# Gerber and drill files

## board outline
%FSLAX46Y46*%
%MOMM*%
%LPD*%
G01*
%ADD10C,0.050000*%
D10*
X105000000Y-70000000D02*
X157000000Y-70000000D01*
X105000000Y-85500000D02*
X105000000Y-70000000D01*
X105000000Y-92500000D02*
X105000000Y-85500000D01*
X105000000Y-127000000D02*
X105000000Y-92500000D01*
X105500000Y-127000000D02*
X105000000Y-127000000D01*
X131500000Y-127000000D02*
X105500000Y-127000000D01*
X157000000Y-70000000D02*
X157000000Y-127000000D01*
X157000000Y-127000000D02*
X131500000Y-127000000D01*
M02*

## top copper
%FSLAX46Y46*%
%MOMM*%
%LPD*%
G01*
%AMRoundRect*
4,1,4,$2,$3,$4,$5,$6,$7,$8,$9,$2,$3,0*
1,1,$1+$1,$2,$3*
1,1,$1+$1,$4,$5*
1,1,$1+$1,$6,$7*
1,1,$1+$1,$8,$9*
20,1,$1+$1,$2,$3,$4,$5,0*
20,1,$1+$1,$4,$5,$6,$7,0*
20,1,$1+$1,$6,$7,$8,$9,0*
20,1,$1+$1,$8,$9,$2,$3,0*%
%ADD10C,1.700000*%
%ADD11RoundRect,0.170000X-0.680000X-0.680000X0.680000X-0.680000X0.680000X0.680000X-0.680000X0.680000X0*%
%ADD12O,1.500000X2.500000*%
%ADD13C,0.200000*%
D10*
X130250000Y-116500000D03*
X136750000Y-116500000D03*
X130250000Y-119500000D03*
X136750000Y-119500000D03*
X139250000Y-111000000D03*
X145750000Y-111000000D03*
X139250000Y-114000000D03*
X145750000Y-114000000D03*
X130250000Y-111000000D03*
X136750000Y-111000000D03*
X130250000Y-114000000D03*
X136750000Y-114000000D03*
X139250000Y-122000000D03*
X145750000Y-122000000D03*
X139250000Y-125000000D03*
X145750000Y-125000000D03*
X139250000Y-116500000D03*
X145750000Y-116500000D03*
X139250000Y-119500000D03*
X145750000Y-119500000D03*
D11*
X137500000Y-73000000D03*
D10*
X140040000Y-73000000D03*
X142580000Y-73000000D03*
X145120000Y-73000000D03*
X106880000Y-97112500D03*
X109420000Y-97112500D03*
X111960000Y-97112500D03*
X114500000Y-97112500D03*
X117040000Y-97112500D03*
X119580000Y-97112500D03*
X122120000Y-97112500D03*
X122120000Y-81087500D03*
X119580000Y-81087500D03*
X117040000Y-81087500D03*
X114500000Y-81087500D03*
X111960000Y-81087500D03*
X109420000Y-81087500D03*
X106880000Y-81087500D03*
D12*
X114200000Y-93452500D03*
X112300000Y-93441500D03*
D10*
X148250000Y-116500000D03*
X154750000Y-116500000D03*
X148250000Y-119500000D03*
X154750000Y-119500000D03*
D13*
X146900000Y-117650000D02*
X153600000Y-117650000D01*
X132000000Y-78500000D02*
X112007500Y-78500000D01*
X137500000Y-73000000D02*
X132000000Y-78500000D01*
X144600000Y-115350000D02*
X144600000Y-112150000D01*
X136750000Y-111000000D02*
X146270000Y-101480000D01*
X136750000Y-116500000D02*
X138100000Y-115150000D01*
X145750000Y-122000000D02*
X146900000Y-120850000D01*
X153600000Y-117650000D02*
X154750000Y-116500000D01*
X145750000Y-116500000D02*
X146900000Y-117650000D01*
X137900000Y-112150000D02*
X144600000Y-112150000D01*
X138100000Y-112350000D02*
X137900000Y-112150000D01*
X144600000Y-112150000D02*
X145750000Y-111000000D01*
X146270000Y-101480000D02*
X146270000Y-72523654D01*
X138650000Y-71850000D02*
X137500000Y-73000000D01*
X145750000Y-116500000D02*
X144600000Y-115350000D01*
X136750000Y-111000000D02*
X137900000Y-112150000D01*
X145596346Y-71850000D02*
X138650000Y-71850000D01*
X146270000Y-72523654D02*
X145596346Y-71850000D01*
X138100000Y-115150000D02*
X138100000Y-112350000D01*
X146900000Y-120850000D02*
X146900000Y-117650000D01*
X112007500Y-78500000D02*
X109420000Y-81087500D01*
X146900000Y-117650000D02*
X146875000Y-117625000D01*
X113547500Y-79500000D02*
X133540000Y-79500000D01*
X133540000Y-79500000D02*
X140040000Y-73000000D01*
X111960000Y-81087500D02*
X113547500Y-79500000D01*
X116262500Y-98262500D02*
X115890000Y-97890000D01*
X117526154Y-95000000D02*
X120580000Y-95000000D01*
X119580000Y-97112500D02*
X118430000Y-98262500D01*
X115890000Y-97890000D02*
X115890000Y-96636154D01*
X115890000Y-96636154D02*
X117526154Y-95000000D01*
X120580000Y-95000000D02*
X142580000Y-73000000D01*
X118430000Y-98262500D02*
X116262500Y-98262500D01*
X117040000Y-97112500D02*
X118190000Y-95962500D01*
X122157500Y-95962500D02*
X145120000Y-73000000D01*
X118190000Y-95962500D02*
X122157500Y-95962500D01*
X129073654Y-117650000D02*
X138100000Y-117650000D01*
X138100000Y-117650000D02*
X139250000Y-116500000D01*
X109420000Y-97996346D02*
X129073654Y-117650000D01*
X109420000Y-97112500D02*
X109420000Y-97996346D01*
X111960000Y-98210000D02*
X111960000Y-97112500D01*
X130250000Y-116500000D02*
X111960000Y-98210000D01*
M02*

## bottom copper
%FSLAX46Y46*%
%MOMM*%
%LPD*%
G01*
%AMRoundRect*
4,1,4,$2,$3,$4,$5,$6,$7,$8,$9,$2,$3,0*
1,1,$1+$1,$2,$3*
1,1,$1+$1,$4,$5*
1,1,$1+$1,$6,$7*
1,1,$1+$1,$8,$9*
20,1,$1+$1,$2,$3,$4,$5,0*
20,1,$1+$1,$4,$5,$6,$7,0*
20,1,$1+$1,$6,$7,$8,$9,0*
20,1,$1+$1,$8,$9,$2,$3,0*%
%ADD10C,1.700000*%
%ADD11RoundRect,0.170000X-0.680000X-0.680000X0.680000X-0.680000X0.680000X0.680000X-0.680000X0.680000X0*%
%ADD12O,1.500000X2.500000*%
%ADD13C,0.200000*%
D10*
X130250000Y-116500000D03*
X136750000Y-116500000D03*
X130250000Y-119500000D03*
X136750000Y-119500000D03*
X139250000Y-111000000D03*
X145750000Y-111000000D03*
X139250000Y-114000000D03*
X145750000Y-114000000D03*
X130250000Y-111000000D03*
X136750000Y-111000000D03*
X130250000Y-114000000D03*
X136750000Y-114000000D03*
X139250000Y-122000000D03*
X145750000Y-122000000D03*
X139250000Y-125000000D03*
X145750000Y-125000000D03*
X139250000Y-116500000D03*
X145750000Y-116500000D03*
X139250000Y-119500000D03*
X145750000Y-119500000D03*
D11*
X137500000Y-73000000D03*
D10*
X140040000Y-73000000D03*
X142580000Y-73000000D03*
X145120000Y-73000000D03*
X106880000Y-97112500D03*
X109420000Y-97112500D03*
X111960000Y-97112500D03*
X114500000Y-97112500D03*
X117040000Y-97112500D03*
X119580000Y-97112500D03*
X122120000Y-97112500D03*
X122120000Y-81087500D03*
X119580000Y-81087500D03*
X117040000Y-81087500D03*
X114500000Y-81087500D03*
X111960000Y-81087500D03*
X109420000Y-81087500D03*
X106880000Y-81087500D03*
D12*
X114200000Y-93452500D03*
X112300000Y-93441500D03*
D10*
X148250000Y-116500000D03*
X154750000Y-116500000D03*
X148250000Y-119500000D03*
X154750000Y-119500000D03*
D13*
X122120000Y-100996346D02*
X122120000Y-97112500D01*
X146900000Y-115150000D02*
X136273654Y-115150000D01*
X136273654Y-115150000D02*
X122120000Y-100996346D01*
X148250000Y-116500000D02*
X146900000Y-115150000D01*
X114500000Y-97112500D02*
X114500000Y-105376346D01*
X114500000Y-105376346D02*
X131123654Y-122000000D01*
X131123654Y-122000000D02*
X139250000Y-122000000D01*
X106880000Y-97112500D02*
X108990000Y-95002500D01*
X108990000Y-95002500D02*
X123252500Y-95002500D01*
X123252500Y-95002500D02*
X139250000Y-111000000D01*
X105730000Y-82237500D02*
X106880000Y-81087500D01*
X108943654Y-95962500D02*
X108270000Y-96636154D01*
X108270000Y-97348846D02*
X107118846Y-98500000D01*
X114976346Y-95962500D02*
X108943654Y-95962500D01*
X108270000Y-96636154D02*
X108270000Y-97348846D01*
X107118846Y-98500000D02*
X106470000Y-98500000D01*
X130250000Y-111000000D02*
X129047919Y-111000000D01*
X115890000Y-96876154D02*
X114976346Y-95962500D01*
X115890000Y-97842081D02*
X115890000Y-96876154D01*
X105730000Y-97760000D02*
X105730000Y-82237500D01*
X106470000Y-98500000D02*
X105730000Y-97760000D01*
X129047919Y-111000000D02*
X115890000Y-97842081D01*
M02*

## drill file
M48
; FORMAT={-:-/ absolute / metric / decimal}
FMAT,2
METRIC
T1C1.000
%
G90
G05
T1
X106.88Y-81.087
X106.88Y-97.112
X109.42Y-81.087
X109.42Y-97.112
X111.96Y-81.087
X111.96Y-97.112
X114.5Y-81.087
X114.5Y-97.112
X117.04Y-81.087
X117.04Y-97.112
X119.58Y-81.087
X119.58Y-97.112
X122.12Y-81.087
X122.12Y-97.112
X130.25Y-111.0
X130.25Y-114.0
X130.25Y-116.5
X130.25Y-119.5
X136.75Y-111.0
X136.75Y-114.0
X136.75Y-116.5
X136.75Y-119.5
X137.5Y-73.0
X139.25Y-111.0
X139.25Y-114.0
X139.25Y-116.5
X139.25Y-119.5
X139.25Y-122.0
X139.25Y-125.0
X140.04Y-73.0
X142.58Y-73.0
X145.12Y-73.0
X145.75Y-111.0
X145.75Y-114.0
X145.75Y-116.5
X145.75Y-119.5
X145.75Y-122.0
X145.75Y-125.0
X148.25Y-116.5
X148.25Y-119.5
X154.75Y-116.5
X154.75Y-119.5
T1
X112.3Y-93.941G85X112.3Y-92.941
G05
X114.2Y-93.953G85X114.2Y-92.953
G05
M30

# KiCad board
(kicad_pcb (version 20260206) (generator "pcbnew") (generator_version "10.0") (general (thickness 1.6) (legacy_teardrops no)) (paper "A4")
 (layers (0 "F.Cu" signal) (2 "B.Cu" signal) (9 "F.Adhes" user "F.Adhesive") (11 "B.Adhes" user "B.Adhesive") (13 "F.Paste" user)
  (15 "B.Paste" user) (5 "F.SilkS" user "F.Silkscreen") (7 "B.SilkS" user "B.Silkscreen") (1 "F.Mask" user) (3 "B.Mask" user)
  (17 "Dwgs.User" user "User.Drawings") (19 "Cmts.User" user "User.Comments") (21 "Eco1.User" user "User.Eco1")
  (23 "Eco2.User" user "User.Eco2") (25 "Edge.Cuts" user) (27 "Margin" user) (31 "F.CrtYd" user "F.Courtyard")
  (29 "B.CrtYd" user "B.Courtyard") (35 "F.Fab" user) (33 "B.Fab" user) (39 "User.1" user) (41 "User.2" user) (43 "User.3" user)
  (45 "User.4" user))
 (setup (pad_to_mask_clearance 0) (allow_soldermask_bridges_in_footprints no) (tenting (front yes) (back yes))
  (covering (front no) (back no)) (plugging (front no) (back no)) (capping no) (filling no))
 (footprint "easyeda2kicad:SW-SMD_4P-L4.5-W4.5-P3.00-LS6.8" (layer "F.Cu") (at 133.5 118)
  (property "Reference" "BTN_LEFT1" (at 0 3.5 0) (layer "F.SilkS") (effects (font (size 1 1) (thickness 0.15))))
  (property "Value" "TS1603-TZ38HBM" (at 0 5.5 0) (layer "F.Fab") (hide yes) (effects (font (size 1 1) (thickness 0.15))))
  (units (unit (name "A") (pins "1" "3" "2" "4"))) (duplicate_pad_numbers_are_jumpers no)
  (pad "1" thru_hole circle (at -3.25 -1.5) (size 1.7 1.7) (drill 1) (layers "*.Cu" "*.Mask") (remove_unused_layers no)
   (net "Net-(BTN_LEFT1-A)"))
  (pad "2" thru_hole circle (at 3.25 -1.5) (size 1.7 1.7) (drill 1) (layers "*.Cu" "*.Mask") (remove_unused_layers no) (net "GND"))
  (pad "3" thru_hole circle (at -3.25 1.5) (size 1.7 1.7) (drill 1) (layers "*.Cu" "*.Mask") (remove_unused_layers no)
   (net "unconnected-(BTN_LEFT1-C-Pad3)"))
  (pad "4" thru_hole circle (at 3.25 1.5) (size 1.7 1.7) (drill 1) (layers "*.Cu" "*.Mask") (remove_unused_layers no)
   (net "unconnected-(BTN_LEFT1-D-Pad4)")))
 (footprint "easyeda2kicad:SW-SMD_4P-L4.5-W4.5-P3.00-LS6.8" (layer "F.Cu") (at 142.5 112.5)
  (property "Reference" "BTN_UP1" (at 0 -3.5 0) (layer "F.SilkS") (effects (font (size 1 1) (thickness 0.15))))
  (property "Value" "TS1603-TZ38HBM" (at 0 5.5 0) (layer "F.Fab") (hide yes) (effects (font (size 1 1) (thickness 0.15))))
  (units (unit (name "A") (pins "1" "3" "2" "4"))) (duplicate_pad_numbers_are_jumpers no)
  (pad "1" thru_hole circle (at -3.25 -1.5) (size 1.7 1.7) (drill 1) (layers "*.Cu" "*.Mask") (remove_unused_layers no)
   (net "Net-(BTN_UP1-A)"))
  (pad "2" thru_hole circle (at 3.25 -1.5) (size 1.7 1.7) (drill 1) (layers "*.Cu" "*.Mask") (remove_unused_layers no) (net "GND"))
  (pad "3" thru_hole circle (at -3.25 1.5) (size 1.7 1.7) (drill 1) (layers "*.Cu" "*.Mask") (remove_unused_layers no)
   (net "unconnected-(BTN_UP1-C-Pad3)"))
  (pad "4" thru_hole circle (at 3.25 1.5) (size 1.7 1.7) (drill 1) (layers "*.Cu" "*.Mask") (remove_unused_layers no)
   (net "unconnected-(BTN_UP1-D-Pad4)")))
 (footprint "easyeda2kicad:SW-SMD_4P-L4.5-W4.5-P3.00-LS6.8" (layer "F.Cu") (at 133.5 112.5)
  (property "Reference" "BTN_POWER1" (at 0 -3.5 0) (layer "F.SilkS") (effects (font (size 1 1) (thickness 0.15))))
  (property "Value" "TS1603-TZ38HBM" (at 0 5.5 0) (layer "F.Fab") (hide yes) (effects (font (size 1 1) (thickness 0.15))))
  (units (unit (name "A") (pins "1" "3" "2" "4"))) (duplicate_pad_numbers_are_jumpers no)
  (pad "1" thru_hole circle (at -3.25 -1.5) (size 1.7 1.7) (drill 1) (layers "*.Cu" "*.Mask") (remove_unused_layers no)
   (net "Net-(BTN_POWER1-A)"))
  (pad "2" thru_hole circle (at 3.25 -1.5) (size 1.7 1.7) (drill 1) (layers "*.Cu" "*.Mask") (remove_unused_layers no) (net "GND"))
  (pad "3" thru_hole circle (at -3.25 1.5) (size 1.7 1.7) (drill 1) (layers "*.Cu" "*.Mask") (remove_unused_layers no)
   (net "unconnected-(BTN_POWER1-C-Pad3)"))
  (pad "4" thru_hole circle (at 3.25 1.5) (size 1.7 1.7) (drill 1) (layers "*.Cu" "*.Mask") (remove_unused_layers no)
   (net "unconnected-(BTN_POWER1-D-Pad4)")))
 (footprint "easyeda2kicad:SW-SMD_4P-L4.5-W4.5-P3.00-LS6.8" (layer "F.Cu") (at 142.5 123.5)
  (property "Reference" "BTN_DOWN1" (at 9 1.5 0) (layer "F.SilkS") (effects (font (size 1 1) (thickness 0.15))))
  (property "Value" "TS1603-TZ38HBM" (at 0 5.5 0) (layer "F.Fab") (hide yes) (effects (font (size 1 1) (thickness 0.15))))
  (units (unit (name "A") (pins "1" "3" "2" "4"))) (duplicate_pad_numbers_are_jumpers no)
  (pad "1" thru_hole circle (at -3.25 -1.5) (size 1.7 1.7) (drill 1) (layers "*.Cu" "*.Mask") (remove_unused_layers no)
   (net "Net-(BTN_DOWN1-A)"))
  (pad "2" thru_hole circle (at 3.25 -1.5) (size 1.7 1.7) (drill 1) (layers "*.Cu" "*.Mask") (remove_unused_layers no) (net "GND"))
  (pad "3" thru_hole circle (at -3.25 1.5) (size 1.7 1.7) (drill 1) (layers "*.Cu" "*.Mask") (remove_unused_layers no)
   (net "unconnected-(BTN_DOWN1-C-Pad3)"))
  (pad "4" thru_hole circle (at 3.25 1.5) (size 1.7 1.7) (drill 1) (layers "*.Cu" "*.Mask") (remove_unused_layers no)
   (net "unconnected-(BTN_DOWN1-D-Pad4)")))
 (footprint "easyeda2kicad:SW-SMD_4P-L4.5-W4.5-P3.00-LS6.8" (layer "F.Cu") (at 142.5 118)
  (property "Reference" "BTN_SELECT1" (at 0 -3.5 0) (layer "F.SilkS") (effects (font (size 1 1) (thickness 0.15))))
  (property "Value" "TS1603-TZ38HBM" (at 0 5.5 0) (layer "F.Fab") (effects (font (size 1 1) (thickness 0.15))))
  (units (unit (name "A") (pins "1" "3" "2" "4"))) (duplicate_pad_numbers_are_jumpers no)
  (pad "1" thru_hole circle (at -3.25 -1.5) (size 1.7 1.7) (drill 1) (layers "*.Cu" "*.Mask") (remove_unused_layers no)
   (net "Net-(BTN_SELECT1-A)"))
  (pad "2" thru_hole circle (at 3.25 -1.5) (size 1.7 1.7) (drill 1) (layers "*.Cu" "*.Mask") (remove_unused_layers no) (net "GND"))
  (pad "3" thru_hole circle (at -3.25 1.5) (size 1.7 1.7) (drill 1) (layers "*.Cu" "*.Mask") (remove_unused_layers no)
   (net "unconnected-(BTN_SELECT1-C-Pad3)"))
  (pad "4" thru_hole circle (at 3.25 1.5) (size 1.7 1.7) (drill 1) (layers "*.Cu" "*.Mask") (remove_unused_layers no)
   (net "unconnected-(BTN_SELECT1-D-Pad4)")))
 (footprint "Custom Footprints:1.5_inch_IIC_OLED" (layer "F.Cu") (at 137.5 73)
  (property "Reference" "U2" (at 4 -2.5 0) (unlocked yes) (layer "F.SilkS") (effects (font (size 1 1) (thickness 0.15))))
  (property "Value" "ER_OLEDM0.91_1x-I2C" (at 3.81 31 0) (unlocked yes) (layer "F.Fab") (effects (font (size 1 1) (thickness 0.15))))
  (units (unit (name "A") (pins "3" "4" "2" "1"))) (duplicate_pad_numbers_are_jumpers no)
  (pad "1" thru_hole roundrect (at 0 0) (size 1.7 1.7) (drill 1) (layers "*.Cu" "*.Mask") (remove_unused_layers no) (roundrect_rratio 0.1)
   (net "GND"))
  (pad "2" thru_hole circle (at 2.54 0) (size 1.7 1.7) (drill 1) (layers "*.Cu" "*.Mask") (remove_unused_layers no) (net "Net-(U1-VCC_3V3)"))
  (pad "3" thru_hole circle (at 5.08 0) (size 1.7 1.7) (drill 1) (layers "*.Cu" "*.Mask") (remove_unused_layers no) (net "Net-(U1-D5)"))
  (pad "4" thru_hole circle (at 7.62 0) (size 1.7 1.7) (drill 1) (layers "*.Cu" "*.Mask") (remove_unused_layers no) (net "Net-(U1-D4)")))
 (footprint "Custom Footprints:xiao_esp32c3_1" (layer "F.Cu") (at 116.3 88.5125 90)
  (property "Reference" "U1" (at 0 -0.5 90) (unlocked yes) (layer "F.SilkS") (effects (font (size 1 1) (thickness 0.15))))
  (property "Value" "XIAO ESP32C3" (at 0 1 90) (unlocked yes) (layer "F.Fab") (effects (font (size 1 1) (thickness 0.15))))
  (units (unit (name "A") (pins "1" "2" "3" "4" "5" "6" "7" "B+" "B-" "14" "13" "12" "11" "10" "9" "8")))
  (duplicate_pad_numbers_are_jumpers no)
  (pad "1" thru_hole circle (at -8.6 -9.42 90) (size 1.7 1.7) (drill 1) (layers "*.Cu" "F.Mask" "F.Paste") (remove_unused_layers no)
   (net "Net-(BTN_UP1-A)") (thermal_bridge_angle 90))
  (pad "2" thru_hole circle (at -8.6 -6.88 90) (size 1.7 1.7) (drill 1) (layers "*.Cu" "*.Mask") (remove_unused_layers no)
   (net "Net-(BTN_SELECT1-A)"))
  (pad "3" thru_hole circle (at -8.6 -4.34 90) (size 1.7 1.7) (drill 1) (layers "*.Cu" "*.Mask") (remove_unused_layers no)
   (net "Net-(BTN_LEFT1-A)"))
  (pad "4" thru_hole circle (at -8.6 -1.8 90) (size 1.7 1.7) (drill 1) (layers "*.Cu" "*.Mask") (remove_unused_layers no)
   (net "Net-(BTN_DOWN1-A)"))
  (pad "5" thru_hole circle (at -8.6 0.74 90) (size 1.7 1.7) (drill 1) (layers "*.Cu" "*.Mask") (remove_unused_layers no)
   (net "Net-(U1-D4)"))
  (pad "6" thru_hole circle (at -8.6 3.28 90) (size 1.7 1.7) (drill 1) (layers "*.Cu" "*.Mask") (remove_unused_layers no)
   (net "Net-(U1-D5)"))
  (pad "7" thru_hole circle (at -8.6 5.82 90) (size 1.7 1.7) (drill 1) (layers "*.Cu" "*.Mask") (remove_unused_layers no)
   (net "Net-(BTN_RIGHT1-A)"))
  (pad "8" thru_hole circle (at 7.425 5.82 90) (size 1.7 1.7) (drill 1) (layers "*.Cu" "*.Mask") (remove_unused_layers no)
   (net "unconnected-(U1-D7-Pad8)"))
  (pad "9" thru_hole circle (at 7.425 3.28 90) (size 1.7 1.7) (drill 1) (layers "*.Cu" "*.Mask") (remove_unused_layers no)
   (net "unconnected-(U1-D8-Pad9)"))
  (pad "10" thru_hole circle (at 7.425 0.74 90) (size 1.7 1.7) (drill 1) (layers "*.Cu" "*.Mask") (remove_unused_layers no)
   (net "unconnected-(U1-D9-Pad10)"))
  (pad "11" thru_hole circle (at 7.425 -1.8 90) (size 1.7 1.7) (drill 1) (layers "*.Cu" "*.Mask") (remove_unused_layers no)
   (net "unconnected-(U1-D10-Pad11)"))
  (pad "12" thru_hole circle (at 7.425 -4.34 90) (size 1.7 1.7) (drill 1) (layers "*.Cu" "*.Mask") (remove_unused_layers no)
   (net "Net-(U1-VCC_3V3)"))
  (pad "13" thru_hole circle (at 7.425 -6.88 90) (size 1.7 1.7) (drill 1) (layers "*.Cu" "*.Mask") (remove_unused_layers no) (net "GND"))
  (pad "14" thru_hole circle (at 7.425 -9.42 90) (size 1.7 1.7) (drill 1) (layers "*.Cu" "F.Mask" "F.Paste") (remove_unused_layers no)
   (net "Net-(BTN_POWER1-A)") (thermal_bridge_angle 90))
  (pad "B+" thru_hole oval (at -4.94 -2.1 90) (size 2.5 1.5) (drill oval 2 1) (layers "*.Cu" "*.Mask") (remove_unused_layers no)
   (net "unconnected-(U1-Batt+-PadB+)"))
  (pad "B-" thru_hole oval (at -4.929 -4 90) (size 2.5 1.5) (drill oval 2 1) (layers "*.Cu" "*.Mask") (remove_unused_layers no)
   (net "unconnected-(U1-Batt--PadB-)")))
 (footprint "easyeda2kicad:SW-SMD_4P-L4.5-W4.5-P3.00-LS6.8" (layer "F.Cu") (at 151.5 118)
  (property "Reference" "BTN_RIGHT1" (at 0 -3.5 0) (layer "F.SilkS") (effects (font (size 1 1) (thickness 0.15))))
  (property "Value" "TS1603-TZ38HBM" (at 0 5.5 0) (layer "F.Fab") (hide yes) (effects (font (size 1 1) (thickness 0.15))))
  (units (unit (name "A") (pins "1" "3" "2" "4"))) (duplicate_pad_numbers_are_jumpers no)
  (pad "1" thru_hole circle (at -3.25 -1.5) (size 1.7 1.7) (drill 1) (layers "*.Cu" "*.Mask") (remove_unused_layers no)
   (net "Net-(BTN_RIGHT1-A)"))
  (pad "2" thru_hole circle (at 3.25 -1.5) (size 1.7 1.7) (drill 1) (layers "*.Cu" "*.Mask") (remove_unused_layers no) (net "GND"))
  (pad "3" thru_hole circle (at -3.25 1.5) (size 1.7 1.7) (drill 1) (layers "*.Cu" "*.Mask") (remove_unused_layers no)
   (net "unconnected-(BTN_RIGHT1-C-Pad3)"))
  (pad "4" thru_hole circle (at 3.25 1.5) (size 1.7 1.7) (drill 1) (layers "*.Cu" "*.Mask") (remove_unused_layers no)
   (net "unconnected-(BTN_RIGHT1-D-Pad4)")))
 (gr_line (start 105 70) (end 157 70) (stroke (width 0.05) (type default)) (layer "Edge.Cuts"))
 (gr_line (start 105 85.5) (end 105 70) (stroke (width 0.05) (type default)) (layer "Edge.Cuts"))
 (gr_line (start 105 92.5) (end 105 85.5) (stroke (width 0.05) (type default)) (layer "Edge.Cuts"))
 (gr_line (start 105 127) (end 105 92.5) (stroke (width 0.05) (type default)) (layer "Edge.Cuts"))
 (gr_line (start 105.5 127) (end 105 127) (stroke (width 0.05) (type default)) (layer "Edge.Cuts"))
 (gr_line (start 131.5 127) (end 105.5 127) (stroke (width 0.05) (type default)) (layer "Edge.Cuts"))
 (gr_line (start 157 70) (end 157 127) (stroke (width 0.05) (type default)) (layer "Edge.Cuts"))
 (gr_line (start 157 127) (end 131.5 127) (stroke (width 0.05) (type default)) (layer "Edge.Cuts"))
 (segment (start 146.9 117.65) (end 153.6 117.65) (width 0.2) (layer "F.Cu") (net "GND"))
 (segment (start 132 78.5) (end 112.0075 78.5) (width 0.2) (layer "F.Cu") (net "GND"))
 (segment (start 137.5 73) (end 132 78.5) (width 0.2) (layer "F.Cu") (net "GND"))
 (segment (start 144.6 115.35) (end 144.6 112.15) (width 0.2) (layer "F.Cu") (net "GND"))
 (segment (start 136.75 111) (end 146.27 101.48) (width 0.2) (layer "F.Cu") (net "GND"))
 (segment (start 136.75 116.5) (end 138.1 115.15) (width 0.2) (layer "F.Cu") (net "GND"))
 (segment (start 145.75 122) (end 146.9 120.85) (width 0.2) (layer "F.Cu") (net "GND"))
 (segment (start 153.6 117.65) (end 154.75 116.5) (width 0.2) (layer "F.Cu") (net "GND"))
 (segment (start 145.75 116.5) (end 146.9 117.65) (width 0.2) (layer "F.Cu") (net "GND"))
 (segment (start 137.9 112.15) (end 144.6 112.15) (width 0.2) (layer "F.Cu") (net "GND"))
 (segment (start 138.1 112.35) (end 137.9 112.15) (width 0.2) (layer "F.Cu") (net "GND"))
 (segment (start 144.6 112.15) (end 145.75 111) (width 0.2) (layer "F.Cu") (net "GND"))
 (segment (start 146.27 101.48) (end 146.27 72.523654) (width 0.2) (layer "F.Cu") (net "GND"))
 (segment (start 138.65 71.85) (end 137.5 73) (width 0.2) (layer "F.Cu") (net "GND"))
 (segment (start 145.75 116.5) (end 144.6 115.35) (width 0.2) (layer "F.Cu") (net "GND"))
 (segment (start 136.75 111) (end 137.9 112.15) (width 0.2) (layer "F.Cu") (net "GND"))
 (segment (start 145.596346 71.85) (end 138.65 71.85) (width 0.2) (layer "F.Cu") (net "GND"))
 (segment (start 146.27 72.523654) (end 145.596346 71.85) (width 0.2) (layer "F.Cu") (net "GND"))
 (segment (start 138.1 115.15) (end 138.1 112.35) (width 0.2) (layer "F.Cu") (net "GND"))
 (segment (start 146.9 120.85) (end 146.9 117.65) (width 0.2) (layer "F.Cu") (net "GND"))
 (segment (start 112.0075 78.5) (end 109.42 81.0875) (width 0.2) (layer "F.Cu") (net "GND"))
 (segment (start 146.9 117.65) (end 146.875 117.625) (width 0.2) (layer "F.Cu") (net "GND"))
 (segment (start 113.5475 79.5) (end 133.54 79.5) (width 0.2) (layer "F.Cu") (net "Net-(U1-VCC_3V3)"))
 (segment (start 133.54 79.5) (end 140.04 73) (width 0.2) (layer "F.Cu") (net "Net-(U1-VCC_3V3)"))
 (segment (start 111.96 81.0875) (end 113.5475 79.5) (width 0.2) (layer "F.Cu") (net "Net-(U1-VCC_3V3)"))
 (segment (start 116.2625 98.2625) (end 115.89 97.89) (width 0.2) (layer "F.Cu") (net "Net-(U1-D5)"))
 (segment (start 117.526154 95) (end 120.58 95) (width 0.2) (layer "F.Cu") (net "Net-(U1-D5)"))
 (segment (start 119.58 97.1125) (end 118.43 98.2625) (width 0.2) (layer "F.Cu") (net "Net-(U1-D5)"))
 (segment (start 115.89 97.89) (end 115.89 96.636154) (width 0.2) (layer "F.Cu") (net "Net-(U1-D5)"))
 (segment (start 115.89 96.636154) (end 117.526154 95) (width 0.2) (layer "F.Cu") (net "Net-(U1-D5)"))
 (segment (start 120.58 95) (end 142.58 73) (width 0.2) (layer "F.Cu") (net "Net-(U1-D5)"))
 (segment (start 118.43 98.2625) (end 116.2625 98.2625) (width 0.2) (layer "F.Cu") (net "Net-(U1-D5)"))
 (segment (start 117.04 97.1125) (end 118.19 95.9625) (width 0.2) (layer "F.Cu") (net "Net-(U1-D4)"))
 (segment (start 122.1575 95.9625) (end 145.12 73) (width 0.2) (layer "F.Cu") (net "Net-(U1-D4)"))
 (segment (start 118.19 95.9625) (end 122.1575 95.9625) (width 0.2) (layer "F.Cu") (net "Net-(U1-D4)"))
 (segment (start 122.12 100.996346) (end 122.12 97.1125) (width 0.2) (layer "B.Cu") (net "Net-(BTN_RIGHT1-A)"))
 (segment (start 146.9 115.15) (end 136.273654 115.15) (width 0.2) (layer "B.Cu") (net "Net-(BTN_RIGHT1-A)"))
 (segment (start 136.273654 115.15) (end 122.12 100.996346) (width 0.2) (layer "B.Cu") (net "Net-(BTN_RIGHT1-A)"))
 (segment (start 148.25 116.5) (end 146.9 115.15) (width 0.2) (layer "B.Cu") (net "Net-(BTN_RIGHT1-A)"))
 (segment (start 114.5 97.1125) (end 114.5 105.376346) (width 0.2) (layer "B.Cu") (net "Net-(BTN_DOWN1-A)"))
 (segment (start 114.5 105.376346) (end 131.123654 122) (width 0.2) (layer "B.Cu") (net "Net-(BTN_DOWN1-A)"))
 (segment (start 131.123654 122) (end 139.25 122) (width 0.2) (layer "B.Cu") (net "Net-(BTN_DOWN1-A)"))
 (segment (start 129.073654 117.65) (end 138.1 117.65) (width 0.2) (layer "F.Cu") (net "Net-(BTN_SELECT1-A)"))
 (segment (start 138.1 117.65) (end 139.25 116.5) (width 0.2) (layer "F.Cu") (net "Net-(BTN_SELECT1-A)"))
 (segment (start 109.42 97.996346) (end 129.073654 117.65) (width 0.2) (layer "F.Cu") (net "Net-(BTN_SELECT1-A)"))
 (segment (start 109.42 97.1125) (end 109.42 97.996346) (width 0.2) (layer "F.Cu") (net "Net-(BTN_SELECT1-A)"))
 (segment (start 111.96 98.21) (end 111.96 97.1125) (width 0.2) (layer "F.Cu") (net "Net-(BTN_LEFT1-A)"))
 (segment (start 130.25 116.5) (end 111.96 98.21) (width 0.2) (layer "F.Cu") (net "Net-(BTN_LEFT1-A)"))
 (segment (start 106.88 97.1125) (end 108.99 95.0025) (width 0.2) (layer "B.Cu") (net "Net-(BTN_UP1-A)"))
 (segment (start 108.99 95.0025) (end 123.2525 95.0025) (width 0.2) (layer "B.Cu") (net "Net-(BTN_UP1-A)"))
 (segment (start 123.2525 95.0025) (end 139.25 111) (width 0.2) (layer "B.Cu") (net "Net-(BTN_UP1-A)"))
 (segment (start 105.73 82.2375) (end 106.88 81.0875) (width 0.2) (layer "B.Cu") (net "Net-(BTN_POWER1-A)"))
 (segment (start 108.943654 95.9625) (end 108.27 96.636154) (width 0.2) (layer "B.Cu") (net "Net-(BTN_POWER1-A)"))
 (segment (start 108.27 97.348846) (end 107.118846 98.5) (width 0.2) (layer "B.Cu") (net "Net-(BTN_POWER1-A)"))
 (segment (start 114.976346 95.9625) (end 108.943654 95.9625) (width 0.2) (layer "B.Cu") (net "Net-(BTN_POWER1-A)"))
 (segment (start 108.27 96.636154) (end 108.27 97.348846) (width 0.2) (layer "B.Cu") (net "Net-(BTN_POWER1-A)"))
 (segment (start 107.118846 98.5) (end 106.47 98.5) (width 0.2) (layer "B.Cu") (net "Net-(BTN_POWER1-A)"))
 (segment (start 130.25 111) (end 129.047919 111) (width 0.2) (layer "B.Cu") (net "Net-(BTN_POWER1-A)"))
 (segment (start 115.89 96.876154) (end 114.976346 95.9625) (width 0.2) (layer "B.Cu") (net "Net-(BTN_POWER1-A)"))
 (segment (start 115.89 97.842081) (end 115.89 96.876154) (width 0.2) (layer "B.Cu") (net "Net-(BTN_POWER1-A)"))
 (segment (start 105.73 97.76) (end 105.73 82.2375) (width 0.2) (layer "B.Cu") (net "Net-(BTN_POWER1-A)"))
 (segment (start 106.47 98.5) (end 105.73 97.76) (width 0.2) (layer "B.Cu") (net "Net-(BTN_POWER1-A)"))
 (segment (start 129.047919 111) (end 115.89 97.842081) (width 0.2) (layer "B.Cu") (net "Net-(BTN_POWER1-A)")))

